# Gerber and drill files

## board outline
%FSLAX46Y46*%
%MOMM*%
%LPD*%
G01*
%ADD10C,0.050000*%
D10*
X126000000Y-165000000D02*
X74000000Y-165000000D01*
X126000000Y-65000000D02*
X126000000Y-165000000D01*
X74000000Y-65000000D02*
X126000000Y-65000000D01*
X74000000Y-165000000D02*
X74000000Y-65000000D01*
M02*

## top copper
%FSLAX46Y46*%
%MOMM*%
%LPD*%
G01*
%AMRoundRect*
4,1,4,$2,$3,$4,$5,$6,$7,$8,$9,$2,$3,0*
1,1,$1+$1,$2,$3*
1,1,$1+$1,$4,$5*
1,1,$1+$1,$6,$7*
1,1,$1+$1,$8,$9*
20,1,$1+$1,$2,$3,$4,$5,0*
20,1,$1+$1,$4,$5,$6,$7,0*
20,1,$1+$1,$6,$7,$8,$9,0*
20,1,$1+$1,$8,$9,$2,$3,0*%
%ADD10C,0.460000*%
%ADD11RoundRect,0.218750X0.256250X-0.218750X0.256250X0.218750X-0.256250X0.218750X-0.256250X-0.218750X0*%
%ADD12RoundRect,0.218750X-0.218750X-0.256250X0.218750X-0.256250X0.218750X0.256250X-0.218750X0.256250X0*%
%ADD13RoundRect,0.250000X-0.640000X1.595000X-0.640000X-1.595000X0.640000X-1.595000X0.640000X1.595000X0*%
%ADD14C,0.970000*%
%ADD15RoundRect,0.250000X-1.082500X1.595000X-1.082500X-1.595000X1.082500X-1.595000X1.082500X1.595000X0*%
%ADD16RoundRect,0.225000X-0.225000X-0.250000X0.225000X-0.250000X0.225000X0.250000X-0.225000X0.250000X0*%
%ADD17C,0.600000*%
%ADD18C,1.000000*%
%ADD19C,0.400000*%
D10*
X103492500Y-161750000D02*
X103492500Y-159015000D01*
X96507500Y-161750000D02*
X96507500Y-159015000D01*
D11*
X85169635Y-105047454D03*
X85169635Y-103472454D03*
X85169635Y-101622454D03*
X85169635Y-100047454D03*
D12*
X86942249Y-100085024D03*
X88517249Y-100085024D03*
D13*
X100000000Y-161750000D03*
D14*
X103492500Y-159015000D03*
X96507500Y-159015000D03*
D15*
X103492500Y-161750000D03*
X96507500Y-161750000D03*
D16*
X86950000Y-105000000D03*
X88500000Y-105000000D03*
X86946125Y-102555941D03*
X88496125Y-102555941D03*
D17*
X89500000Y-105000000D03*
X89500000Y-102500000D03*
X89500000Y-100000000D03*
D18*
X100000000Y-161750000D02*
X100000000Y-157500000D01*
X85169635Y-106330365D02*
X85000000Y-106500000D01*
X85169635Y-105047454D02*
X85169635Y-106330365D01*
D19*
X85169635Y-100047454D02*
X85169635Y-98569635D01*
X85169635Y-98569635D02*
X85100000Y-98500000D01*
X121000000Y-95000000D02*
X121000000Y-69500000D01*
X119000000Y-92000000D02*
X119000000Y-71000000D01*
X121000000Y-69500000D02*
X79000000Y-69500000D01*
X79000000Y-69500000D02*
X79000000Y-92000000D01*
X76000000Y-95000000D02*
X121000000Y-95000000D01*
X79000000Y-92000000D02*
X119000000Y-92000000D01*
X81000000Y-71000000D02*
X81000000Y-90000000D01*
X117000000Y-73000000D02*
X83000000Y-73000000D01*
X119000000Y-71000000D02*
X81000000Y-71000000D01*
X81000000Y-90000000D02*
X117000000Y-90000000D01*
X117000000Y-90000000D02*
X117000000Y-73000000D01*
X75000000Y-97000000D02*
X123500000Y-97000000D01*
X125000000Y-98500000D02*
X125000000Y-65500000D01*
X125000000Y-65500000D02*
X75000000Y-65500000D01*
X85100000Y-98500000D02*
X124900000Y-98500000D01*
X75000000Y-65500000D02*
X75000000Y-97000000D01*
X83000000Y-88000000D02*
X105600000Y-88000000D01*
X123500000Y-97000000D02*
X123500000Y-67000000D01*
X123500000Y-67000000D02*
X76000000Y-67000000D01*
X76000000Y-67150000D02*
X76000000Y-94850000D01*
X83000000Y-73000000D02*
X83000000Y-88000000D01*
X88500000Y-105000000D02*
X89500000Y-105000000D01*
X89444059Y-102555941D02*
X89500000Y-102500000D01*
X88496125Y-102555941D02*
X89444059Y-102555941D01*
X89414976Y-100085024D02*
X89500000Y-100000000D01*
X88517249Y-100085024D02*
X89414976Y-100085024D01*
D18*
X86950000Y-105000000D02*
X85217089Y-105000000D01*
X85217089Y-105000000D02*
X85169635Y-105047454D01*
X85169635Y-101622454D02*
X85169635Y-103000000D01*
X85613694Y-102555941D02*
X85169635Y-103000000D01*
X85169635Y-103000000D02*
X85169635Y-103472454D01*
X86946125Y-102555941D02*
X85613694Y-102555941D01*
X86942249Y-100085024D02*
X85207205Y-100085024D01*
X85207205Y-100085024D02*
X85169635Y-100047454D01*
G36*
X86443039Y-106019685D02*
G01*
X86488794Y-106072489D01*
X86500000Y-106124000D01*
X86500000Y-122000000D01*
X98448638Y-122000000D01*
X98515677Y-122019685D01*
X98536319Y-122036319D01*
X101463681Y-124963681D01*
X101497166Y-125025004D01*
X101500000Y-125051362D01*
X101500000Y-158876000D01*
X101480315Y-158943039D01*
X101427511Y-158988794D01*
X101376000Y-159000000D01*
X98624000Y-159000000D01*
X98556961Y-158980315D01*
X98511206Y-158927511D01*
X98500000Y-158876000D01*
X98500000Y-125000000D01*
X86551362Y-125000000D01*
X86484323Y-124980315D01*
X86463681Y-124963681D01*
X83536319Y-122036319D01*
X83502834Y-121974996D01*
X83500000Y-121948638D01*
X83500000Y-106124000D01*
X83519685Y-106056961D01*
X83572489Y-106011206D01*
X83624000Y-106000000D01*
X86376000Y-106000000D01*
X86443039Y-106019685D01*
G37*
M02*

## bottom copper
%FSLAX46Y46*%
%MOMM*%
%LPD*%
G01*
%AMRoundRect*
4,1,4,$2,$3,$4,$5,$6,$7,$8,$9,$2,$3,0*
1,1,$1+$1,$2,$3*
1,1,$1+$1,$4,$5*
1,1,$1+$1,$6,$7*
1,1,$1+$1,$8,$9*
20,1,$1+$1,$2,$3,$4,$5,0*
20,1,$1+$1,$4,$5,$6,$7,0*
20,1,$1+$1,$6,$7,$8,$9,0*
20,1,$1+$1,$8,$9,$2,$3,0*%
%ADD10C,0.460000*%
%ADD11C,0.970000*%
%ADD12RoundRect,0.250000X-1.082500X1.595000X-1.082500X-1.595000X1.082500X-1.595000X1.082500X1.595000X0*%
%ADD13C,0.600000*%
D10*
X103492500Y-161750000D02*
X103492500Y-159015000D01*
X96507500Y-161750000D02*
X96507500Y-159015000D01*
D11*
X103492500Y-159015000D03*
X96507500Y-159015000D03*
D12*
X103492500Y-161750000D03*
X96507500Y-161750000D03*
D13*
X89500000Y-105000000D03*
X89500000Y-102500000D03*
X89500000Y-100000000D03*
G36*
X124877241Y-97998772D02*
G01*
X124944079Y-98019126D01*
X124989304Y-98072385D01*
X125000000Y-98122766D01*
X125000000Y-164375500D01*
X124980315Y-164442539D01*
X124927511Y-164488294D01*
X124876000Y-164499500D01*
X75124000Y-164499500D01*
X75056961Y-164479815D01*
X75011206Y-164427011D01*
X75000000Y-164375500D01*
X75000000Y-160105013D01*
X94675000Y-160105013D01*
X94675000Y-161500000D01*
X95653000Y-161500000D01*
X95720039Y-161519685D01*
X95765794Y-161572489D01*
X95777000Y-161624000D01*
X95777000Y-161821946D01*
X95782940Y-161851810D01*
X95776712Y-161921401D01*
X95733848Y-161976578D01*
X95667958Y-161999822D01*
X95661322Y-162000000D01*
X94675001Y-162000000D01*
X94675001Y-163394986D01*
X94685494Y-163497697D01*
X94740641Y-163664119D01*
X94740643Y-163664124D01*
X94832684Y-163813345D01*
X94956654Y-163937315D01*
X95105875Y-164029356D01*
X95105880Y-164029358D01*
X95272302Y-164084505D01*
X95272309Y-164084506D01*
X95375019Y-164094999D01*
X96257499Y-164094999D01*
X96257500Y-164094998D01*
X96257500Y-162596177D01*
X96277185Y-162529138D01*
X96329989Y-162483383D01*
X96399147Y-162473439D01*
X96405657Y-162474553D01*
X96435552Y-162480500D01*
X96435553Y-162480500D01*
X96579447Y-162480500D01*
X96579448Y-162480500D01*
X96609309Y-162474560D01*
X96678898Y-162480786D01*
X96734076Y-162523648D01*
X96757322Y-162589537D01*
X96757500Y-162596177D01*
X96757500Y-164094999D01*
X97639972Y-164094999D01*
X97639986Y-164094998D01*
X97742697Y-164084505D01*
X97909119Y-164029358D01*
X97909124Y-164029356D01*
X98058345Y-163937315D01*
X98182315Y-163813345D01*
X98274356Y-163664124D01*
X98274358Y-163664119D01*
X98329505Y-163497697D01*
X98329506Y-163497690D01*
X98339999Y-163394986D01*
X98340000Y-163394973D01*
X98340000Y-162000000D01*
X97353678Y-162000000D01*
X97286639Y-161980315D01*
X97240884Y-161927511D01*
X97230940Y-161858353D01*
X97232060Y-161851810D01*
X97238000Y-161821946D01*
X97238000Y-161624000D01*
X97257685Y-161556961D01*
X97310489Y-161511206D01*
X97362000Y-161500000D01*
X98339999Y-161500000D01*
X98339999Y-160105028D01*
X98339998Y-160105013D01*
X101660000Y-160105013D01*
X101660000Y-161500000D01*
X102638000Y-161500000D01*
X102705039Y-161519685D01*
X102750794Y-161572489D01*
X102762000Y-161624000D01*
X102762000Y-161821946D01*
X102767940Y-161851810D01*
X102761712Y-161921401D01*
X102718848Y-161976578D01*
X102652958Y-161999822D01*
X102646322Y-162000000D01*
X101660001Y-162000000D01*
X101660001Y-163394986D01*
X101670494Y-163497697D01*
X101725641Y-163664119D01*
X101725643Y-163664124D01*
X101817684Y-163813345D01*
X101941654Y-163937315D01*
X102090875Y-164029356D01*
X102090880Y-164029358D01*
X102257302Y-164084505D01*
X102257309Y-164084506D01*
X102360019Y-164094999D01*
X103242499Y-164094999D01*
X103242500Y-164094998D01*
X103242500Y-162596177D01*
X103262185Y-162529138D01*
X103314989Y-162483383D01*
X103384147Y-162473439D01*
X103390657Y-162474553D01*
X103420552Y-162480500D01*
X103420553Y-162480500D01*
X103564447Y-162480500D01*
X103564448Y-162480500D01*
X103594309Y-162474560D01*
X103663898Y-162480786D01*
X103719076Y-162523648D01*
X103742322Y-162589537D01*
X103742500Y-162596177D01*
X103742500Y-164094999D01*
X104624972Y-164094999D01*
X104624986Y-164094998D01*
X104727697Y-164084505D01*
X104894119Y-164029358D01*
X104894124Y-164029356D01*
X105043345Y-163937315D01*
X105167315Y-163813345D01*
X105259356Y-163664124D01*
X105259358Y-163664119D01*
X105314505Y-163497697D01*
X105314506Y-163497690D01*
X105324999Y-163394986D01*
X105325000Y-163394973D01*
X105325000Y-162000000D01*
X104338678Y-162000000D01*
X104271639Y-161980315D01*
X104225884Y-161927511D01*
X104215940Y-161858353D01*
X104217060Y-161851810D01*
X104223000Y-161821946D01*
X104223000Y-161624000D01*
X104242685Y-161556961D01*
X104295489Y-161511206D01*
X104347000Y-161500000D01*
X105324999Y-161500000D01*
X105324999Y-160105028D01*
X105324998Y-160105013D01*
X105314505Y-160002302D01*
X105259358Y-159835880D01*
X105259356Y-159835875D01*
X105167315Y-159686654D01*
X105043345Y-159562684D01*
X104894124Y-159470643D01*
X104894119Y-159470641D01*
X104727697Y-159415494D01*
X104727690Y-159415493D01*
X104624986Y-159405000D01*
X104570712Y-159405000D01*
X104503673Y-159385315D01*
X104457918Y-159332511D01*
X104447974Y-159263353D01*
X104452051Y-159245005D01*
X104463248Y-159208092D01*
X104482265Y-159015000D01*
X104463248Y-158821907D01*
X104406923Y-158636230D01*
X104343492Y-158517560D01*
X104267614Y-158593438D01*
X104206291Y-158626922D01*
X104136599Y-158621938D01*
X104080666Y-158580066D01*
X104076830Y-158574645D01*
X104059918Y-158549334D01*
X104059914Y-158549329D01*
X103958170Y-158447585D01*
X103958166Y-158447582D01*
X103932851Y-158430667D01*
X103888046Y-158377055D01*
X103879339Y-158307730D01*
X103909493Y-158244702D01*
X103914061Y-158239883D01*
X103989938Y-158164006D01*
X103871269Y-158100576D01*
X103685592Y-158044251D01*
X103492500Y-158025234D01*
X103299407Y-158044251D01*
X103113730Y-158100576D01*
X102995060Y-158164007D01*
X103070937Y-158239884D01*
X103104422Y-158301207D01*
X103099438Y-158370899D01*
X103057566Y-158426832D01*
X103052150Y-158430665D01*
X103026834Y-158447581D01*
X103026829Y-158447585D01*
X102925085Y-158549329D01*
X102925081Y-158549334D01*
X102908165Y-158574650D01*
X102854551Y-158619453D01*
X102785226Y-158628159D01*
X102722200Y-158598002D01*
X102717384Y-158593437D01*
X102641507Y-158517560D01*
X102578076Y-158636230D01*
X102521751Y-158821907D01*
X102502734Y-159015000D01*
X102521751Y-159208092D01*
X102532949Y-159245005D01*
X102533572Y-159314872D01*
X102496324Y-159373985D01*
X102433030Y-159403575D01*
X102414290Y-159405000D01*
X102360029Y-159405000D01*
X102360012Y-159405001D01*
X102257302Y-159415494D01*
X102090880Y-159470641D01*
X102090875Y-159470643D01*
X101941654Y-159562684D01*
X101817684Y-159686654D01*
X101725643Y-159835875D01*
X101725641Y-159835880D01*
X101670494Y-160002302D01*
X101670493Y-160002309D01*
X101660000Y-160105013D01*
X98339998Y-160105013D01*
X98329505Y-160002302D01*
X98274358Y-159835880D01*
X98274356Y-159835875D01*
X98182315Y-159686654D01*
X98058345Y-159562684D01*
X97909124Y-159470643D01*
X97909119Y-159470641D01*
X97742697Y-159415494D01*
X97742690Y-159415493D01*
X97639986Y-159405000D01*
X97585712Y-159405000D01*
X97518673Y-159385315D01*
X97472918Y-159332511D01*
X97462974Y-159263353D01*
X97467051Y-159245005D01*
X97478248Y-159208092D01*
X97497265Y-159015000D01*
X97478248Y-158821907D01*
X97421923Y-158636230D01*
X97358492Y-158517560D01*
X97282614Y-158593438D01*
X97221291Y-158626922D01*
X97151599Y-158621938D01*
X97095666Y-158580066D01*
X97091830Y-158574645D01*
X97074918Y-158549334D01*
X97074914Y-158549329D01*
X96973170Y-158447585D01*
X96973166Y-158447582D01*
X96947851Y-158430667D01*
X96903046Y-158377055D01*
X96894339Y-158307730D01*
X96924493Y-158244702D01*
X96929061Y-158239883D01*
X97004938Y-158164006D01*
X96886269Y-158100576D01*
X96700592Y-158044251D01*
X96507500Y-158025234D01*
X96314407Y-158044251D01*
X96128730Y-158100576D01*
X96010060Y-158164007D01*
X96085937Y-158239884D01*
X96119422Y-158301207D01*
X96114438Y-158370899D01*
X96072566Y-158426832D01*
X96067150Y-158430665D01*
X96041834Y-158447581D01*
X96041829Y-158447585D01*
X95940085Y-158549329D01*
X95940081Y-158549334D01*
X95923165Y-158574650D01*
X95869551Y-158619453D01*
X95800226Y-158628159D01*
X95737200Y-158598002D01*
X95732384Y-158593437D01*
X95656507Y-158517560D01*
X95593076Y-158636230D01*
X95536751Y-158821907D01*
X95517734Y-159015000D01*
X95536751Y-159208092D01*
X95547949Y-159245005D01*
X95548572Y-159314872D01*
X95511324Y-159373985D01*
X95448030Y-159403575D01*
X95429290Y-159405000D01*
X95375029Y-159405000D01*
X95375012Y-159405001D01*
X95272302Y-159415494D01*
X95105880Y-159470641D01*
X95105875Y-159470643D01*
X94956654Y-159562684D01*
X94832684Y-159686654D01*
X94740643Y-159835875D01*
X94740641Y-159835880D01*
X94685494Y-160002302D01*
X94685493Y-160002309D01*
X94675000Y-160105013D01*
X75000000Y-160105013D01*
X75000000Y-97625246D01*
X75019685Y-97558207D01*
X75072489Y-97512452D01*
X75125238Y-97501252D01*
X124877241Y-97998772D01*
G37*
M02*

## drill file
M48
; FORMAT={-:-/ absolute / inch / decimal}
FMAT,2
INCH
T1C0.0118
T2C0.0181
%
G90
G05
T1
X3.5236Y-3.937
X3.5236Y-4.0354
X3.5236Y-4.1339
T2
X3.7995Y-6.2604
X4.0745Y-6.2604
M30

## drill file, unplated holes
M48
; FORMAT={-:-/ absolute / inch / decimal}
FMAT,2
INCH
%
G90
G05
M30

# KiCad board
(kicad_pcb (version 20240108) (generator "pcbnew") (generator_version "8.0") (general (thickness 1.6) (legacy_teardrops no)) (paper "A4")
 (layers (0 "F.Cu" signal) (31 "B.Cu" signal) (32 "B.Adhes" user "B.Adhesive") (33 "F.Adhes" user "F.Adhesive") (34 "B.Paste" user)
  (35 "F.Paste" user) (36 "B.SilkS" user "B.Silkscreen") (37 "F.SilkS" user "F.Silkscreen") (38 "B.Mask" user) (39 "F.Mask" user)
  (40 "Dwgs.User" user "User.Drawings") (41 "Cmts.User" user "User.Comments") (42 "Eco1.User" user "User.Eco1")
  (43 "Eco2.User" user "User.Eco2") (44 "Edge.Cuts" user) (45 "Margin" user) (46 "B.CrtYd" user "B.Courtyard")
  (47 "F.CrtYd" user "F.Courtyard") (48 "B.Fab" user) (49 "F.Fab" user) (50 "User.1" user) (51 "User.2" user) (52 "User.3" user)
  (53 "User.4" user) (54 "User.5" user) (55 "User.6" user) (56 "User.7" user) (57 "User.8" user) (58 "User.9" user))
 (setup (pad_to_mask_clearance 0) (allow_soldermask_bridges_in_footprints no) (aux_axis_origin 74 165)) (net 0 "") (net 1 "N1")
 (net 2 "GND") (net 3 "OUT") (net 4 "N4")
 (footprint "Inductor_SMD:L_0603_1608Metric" (layer "F.Cu") (at 87.729749 100.085024)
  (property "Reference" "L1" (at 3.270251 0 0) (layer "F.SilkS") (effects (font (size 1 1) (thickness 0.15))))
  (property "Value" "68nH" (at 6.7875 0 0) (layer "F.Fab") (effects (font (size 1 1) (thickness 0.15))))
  (pad "1" smd roundrect (at -0.7875 0) (size 0.875 0.95) (layers "F.Cu" "F.Paste" "F.Mask") (roundrect_rratio 0.25) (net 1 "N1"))
  (pad "2" smd roundrect (at 0.7875 0) (size 0.875 0.95) (layers "F.Cu" "F.Paste" "F.Mask") (roundrect_rratio 0.25) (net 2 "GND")))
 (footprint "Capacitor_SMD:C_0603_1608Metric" (layer "F.Cu") (at 87.725 105)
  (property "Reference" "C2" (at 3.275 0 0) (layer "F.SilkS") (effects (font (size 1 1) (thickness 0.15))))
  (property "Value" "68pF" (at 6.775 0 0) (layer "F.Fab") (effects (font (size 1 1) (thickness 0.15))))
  (pad "1" smd roundrect (at -0.775 0) (size 0.9 0.95) (layers "F.Cu" "F.Paste" "F.Mask") (roundrect_rratio 0.25) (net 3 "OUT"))
  (pad "2" smd roundrect (at 0.775 0) (size 0.9 0.95) (layers "F.Cu" "F.Paste" "F.Mask") (roundrect_rratio 0.25) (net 2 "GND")))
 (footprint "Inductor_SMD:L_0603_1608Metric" (layer "F.Cu") (at 85.169635 104.259954 90)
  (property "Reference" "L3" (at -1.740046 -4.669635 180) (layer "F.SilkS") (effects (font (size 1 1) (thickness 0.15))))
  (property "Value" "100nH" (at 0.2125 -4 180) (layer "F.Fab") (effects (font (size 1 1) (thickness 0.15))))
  (pad "1" smd roundrect (at -0.7875 0 90) (size 0.875 0.95) (layers "F.Cu" "F.Paste" "F.Mask") (roundrect_rratio 0.25) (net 3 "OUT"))
  (pad "2" smd roundrect (at 0.7875 0 90) (size 0.875 0.95) (layers "F.Cu" "F.Paste" "F.Mask") (roundrect_rratio 0.25) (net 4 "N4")))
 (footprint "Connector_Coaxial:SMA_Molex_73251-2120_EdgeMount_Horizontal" (layer "F.Cu") (at 100 162 -90)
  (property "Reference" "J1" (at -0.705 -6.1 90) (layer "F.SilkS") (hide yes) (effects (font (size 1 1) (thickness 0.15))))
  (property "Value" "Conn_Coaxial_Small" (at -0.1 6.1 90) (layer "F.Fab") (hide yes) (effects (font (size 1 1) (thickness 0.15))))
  (fp_line (start -0.25 3.4925) (end -2.985 3.4925) (stroke (width 0.46) (type default)) (layer "F.Cu"))
  (fp_line (start -0.25 -3.4925) (end -2.985 -3.4925) (stroke (width 0.46) (type default)) (layer "F.Cu"))
  (fp_line (start -0.25 3.4925) (end -2.985 3.4925) (stroke (width 0.46) (type default)) (layer "B.Cu"))
  (fp_line (start -0.25 -3.4925) (end -2.985 -3.4925) (stroke (width 0.46) (type default)) (layer "B.Cu"))
  (pad "1" smd roundrect (at -0.25 0 270) (size 3.69 1.78) (layers "F.Cu" "F.Paste" "F.Mask") (roundrect_rratio 0.1404494382) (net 3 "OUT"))
  (pad "2" thru_hole circle (at -2.985 -3.4925 270) (size 0.97 0.97) (drill 0.46) (layers "*.Cu") (remove_unused_layers no) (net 2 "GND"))
  (pad "2" thru_hole circle (at -2.985 3.4925 270) (size 0.97 0.97) (drill 0.46) (layers "*.Cu") (remove_unused_layers no) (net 2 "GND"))
  (pad "2" smd roundrect (at -0.25 -3.4925 270) (size 3.69 2.665) (layers "F.Cu" "F.Paste" "F.Mask") (roundrect_rratio 0.09380863039)
   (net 2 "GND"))
  (pad "2" smd roundrect (at -0.25 -3.4925 270) (size 3.69 2.665) (layers "B.Cu" "B.Paste" "B.Mask") (roundrect_rratio 0.09380863039)
   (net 2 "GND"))
  (pad "2" smd roundrect (at -0.25 3.4925 270) (size 3.69 2.665) (layers "F.Cu" "F.Paste" "F.Mask") (roundrect_rratio 0.09380863039)
   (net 2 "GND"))
  (pad "2" smd roundrect (at -0.25 3.4925 270) (size 3.69 2.665) (layers "B.Cu" "B.Paste" "B.Mask") (roundrect_rratio 0.09380863039)
   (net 2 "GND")))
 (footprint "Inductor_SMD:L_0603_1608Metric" (layer "F.Cu") (at 85.169635 100.834954 90)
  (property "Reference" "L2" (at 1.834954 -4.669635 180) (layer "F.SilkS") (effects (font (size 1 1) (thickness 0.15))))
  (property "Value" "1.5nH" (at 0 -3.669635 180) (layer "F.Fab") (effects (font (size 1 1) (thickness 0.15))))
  (pad "1" smd roundrect (at -0.7875 0 90) (size 0.875 0.95) (layers "F.Cu" "F.Paste" "F.Mask") (roundrect_rratio 0.25) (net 4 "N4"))
  (pad "2" smd roundrect (at 0.7875 0 90) (size 0.875 0.95) (layers "F.Cu" "F.Paste" "F.Mask") (roundrect_rratio 0.25) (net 1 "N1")))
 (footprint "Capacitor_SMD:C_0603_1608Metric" (layer "F.Cu") (at 87.721125 102.555941)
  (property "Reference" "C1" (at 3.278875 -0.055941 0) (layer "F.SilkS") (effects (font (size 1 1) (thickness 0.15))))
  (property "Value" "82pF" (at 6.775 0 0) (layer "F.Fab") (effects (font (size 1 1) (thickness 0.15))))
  (pad "1" smd roundrect (at -0.775 0) (size 0.9 0.95) (layers "F.Cu" "F.Paste" "F.Mask") (roundrect_rratio 0.25) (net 4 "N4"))
  (pad "2" smd roundrect (at 0.775 0) (size 0.9 0.95) (layers "F.Cu" "F.Paste" "F.Mask") (roundrect_rratio 0.25) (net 2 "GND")))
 (gr_line (start 74 65) (end 126 65) (stroke (width 0.05) (type default)) (layer "Edge.Cuts"))
 (gr_line (start 126 65) (end 126 165) (stroke (width 0.05) (type default)) (layer "Edge.Cuts"))
 (gr_line (start 74 165) (end 74 65) (stroke (width 0.05) (type default)) (layer "Edge.Cuts"))
 (gr_line (start 126 165) (end 74 165) (stroke (width 0.05) (type default)) (layer "Edge.Cuts"))
 (segment (start 85.613694 102.555941) (end 85.169635 103) (width 1) (layer "F.Cu") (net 4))
 (segment (start 86.946125 102.555941) (end 85.613694 102.555941) (width 1) (layer "F.Cu") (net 4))
 (segment (start 85.169635 103) (end 85.169635 103.472454) (width 1) (layer "F.Cu") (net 4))
 (segment (start 85.169635 101.622454) (end 85.169635 103) (width 1) (layer "F.Cu") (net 4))
 (segment (start 89.414976 100.085024) (end 89.5 100) (width 0.4) (layer "F.Cu") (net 2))
 (segment (start 88.5 105) (end 89.5 105) (width 0.4) (layer "F.Cu") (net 2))
 (segment (start 89.444059 102.555941) (end 89.5 102.5) (width 0.4) (layer "F.Cu") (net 2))
 (segment (start 88.517249 100.085024) (end 89.414976 100.085024) (width 0.4) (layer "F.Cu") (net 2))
 (segment (start 88.496125 102.555941) (end 89.444059 102.555941) (width 0.4) (layer "F.Cu") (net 2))
 (via (at 89.5 100) (size 0.6) (drill 0.3) (layers "F.Cu" "B.Cu") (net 2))
 (via (at 89.5 105) (size 0.6) (drill 0.3) (layers "F.Cu" "B.Cu") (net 2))
 (via (at 89.5 102.5) (size 0.6) (drill 0.3) (layers "F.Cu" "B.Cu") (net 2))
 (segment (start 85.1 98.5) (end 124.9 98.5) (width 0.4) (layer "F.Cu") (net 1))
 (segment (start 117 90) (end 117 73) (width 0.4) (layer "F.Cu") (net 1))
 (segment (start 125 98.5) (end 125 65.5) (width 0.4) (layer "F.Cu") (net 1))
 (segment (start 76 67.15) (end 76 94.85) (width 0.4) (layer "F.Cu") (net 1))
 (segment (start 83 88) (end 105.6 88) (width 0.4) (layer "F.Cu") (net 1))
 (segment (start 123.5 67) (end 76 67) (width 0.4) (layer "F.Cu") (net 1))
 (segment (start 83 73) (end 83 88) (width 0.4) (layer "F.Cu") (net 1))
 (segment (start 123.5 97) (end 123.5 67) (width 0.4) (layer "F.Cu") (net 1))
 (segment (start 121 95) (end 121 69.5) (width 0.4) (layer "F.Cu") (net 1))
 (segment (start 119 92) (end 119 71) (width 0.4) (layer "F.Cu") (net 1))
 (segment (start 85.169635 98.569635) (end 85.1 98.5) (width 0.4) (layer "F.Cu") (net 1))
 (segment (start 85.207205 100.085024) (end 85.169635 100.047454) (width 1) (layer "F.Cu") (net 1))
 (segment (start 81 71) (end 81 90) (width 0.4) (layer "F.Cu") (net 1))
 (segment (start 75 65.5) (end 75 97) (width 0.4) (layer "F.Cu") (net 1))
 (segment (start 125 65.5) (end 75 65.5) (width 0.4) (layer "F.Cu") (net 1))
 (segment (start 121 69.5) (end 79 69.5) (width 0.4) (layer "F.Cu") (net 1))
 (segment (start 85.169635 100.047454) (end 85.169635 98.569635) (width 0.4) (layer "F.Cu") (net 1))
 (segment (start 81 90) (end 117 90) (width 0.4) (layer "F.Cu") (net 1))
 (segment (start 75 97) (end 123.5 97) (width 0.4) (layer "F.Cu") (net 1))
 (segment (start 79 69.5) (end 79 92) (width 0.4) (layer "F.Cu") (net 1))
 (segment (start 76 95) (end 121 95) (width 0.4) (layer "F.Cu") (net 1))
 (segment (start 79 92) (end 119 92) (width 0.4) (layer "F.Cu") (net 1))
 (segment (start 119 71) (end 81 71) (width 0.4) (layer "F.Cu") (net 1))
 (segment (start 117 73) (end 83 73) (width 0.4) (layer "F.Cu") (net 1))
 (segment (start 86.942249 100.085024) (end 85.207205 100.085024) (width 1) (layer "F.Cu") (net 1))
 (segment (start 85.169635 106.330365) (end 85 106.5) (width 1) (layer "F.Cu") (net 3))
 (segment (start 100 161.75) (end 100 157.5) (width 1) (layer "F.Cu") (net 3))
 (segment (start 85.217089 105) (end 85.169635 105.047454) (width 1) (layer "F.Cu") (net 3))
 (segment (start 86.95 105) (end 85.217089 105) (width 1) (layer "F.Cu") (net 3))
 (segment (start 85.169635 105.047454) (end 85.169635 106.330365) (width 1) (layer "F.Cu") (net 3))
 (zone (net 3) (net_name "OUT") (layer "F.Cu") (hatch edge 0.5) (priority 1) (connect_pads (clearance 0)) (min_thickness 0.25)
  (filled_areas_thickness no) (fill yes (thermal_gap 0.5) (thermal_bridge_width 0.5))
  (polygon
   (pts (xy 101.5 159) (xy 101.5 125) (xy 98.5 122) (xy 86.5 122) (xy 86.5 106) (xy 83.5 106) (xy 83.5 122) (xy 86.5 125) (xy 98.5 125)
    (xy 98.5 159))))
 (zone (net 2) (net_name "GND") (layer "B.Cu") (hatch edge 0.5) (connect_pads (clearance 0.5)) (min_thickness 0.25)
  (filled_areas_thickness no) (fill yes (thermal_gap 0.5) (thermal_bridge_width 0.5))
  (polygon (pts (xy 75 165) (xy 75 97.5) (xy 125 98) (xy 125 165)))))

